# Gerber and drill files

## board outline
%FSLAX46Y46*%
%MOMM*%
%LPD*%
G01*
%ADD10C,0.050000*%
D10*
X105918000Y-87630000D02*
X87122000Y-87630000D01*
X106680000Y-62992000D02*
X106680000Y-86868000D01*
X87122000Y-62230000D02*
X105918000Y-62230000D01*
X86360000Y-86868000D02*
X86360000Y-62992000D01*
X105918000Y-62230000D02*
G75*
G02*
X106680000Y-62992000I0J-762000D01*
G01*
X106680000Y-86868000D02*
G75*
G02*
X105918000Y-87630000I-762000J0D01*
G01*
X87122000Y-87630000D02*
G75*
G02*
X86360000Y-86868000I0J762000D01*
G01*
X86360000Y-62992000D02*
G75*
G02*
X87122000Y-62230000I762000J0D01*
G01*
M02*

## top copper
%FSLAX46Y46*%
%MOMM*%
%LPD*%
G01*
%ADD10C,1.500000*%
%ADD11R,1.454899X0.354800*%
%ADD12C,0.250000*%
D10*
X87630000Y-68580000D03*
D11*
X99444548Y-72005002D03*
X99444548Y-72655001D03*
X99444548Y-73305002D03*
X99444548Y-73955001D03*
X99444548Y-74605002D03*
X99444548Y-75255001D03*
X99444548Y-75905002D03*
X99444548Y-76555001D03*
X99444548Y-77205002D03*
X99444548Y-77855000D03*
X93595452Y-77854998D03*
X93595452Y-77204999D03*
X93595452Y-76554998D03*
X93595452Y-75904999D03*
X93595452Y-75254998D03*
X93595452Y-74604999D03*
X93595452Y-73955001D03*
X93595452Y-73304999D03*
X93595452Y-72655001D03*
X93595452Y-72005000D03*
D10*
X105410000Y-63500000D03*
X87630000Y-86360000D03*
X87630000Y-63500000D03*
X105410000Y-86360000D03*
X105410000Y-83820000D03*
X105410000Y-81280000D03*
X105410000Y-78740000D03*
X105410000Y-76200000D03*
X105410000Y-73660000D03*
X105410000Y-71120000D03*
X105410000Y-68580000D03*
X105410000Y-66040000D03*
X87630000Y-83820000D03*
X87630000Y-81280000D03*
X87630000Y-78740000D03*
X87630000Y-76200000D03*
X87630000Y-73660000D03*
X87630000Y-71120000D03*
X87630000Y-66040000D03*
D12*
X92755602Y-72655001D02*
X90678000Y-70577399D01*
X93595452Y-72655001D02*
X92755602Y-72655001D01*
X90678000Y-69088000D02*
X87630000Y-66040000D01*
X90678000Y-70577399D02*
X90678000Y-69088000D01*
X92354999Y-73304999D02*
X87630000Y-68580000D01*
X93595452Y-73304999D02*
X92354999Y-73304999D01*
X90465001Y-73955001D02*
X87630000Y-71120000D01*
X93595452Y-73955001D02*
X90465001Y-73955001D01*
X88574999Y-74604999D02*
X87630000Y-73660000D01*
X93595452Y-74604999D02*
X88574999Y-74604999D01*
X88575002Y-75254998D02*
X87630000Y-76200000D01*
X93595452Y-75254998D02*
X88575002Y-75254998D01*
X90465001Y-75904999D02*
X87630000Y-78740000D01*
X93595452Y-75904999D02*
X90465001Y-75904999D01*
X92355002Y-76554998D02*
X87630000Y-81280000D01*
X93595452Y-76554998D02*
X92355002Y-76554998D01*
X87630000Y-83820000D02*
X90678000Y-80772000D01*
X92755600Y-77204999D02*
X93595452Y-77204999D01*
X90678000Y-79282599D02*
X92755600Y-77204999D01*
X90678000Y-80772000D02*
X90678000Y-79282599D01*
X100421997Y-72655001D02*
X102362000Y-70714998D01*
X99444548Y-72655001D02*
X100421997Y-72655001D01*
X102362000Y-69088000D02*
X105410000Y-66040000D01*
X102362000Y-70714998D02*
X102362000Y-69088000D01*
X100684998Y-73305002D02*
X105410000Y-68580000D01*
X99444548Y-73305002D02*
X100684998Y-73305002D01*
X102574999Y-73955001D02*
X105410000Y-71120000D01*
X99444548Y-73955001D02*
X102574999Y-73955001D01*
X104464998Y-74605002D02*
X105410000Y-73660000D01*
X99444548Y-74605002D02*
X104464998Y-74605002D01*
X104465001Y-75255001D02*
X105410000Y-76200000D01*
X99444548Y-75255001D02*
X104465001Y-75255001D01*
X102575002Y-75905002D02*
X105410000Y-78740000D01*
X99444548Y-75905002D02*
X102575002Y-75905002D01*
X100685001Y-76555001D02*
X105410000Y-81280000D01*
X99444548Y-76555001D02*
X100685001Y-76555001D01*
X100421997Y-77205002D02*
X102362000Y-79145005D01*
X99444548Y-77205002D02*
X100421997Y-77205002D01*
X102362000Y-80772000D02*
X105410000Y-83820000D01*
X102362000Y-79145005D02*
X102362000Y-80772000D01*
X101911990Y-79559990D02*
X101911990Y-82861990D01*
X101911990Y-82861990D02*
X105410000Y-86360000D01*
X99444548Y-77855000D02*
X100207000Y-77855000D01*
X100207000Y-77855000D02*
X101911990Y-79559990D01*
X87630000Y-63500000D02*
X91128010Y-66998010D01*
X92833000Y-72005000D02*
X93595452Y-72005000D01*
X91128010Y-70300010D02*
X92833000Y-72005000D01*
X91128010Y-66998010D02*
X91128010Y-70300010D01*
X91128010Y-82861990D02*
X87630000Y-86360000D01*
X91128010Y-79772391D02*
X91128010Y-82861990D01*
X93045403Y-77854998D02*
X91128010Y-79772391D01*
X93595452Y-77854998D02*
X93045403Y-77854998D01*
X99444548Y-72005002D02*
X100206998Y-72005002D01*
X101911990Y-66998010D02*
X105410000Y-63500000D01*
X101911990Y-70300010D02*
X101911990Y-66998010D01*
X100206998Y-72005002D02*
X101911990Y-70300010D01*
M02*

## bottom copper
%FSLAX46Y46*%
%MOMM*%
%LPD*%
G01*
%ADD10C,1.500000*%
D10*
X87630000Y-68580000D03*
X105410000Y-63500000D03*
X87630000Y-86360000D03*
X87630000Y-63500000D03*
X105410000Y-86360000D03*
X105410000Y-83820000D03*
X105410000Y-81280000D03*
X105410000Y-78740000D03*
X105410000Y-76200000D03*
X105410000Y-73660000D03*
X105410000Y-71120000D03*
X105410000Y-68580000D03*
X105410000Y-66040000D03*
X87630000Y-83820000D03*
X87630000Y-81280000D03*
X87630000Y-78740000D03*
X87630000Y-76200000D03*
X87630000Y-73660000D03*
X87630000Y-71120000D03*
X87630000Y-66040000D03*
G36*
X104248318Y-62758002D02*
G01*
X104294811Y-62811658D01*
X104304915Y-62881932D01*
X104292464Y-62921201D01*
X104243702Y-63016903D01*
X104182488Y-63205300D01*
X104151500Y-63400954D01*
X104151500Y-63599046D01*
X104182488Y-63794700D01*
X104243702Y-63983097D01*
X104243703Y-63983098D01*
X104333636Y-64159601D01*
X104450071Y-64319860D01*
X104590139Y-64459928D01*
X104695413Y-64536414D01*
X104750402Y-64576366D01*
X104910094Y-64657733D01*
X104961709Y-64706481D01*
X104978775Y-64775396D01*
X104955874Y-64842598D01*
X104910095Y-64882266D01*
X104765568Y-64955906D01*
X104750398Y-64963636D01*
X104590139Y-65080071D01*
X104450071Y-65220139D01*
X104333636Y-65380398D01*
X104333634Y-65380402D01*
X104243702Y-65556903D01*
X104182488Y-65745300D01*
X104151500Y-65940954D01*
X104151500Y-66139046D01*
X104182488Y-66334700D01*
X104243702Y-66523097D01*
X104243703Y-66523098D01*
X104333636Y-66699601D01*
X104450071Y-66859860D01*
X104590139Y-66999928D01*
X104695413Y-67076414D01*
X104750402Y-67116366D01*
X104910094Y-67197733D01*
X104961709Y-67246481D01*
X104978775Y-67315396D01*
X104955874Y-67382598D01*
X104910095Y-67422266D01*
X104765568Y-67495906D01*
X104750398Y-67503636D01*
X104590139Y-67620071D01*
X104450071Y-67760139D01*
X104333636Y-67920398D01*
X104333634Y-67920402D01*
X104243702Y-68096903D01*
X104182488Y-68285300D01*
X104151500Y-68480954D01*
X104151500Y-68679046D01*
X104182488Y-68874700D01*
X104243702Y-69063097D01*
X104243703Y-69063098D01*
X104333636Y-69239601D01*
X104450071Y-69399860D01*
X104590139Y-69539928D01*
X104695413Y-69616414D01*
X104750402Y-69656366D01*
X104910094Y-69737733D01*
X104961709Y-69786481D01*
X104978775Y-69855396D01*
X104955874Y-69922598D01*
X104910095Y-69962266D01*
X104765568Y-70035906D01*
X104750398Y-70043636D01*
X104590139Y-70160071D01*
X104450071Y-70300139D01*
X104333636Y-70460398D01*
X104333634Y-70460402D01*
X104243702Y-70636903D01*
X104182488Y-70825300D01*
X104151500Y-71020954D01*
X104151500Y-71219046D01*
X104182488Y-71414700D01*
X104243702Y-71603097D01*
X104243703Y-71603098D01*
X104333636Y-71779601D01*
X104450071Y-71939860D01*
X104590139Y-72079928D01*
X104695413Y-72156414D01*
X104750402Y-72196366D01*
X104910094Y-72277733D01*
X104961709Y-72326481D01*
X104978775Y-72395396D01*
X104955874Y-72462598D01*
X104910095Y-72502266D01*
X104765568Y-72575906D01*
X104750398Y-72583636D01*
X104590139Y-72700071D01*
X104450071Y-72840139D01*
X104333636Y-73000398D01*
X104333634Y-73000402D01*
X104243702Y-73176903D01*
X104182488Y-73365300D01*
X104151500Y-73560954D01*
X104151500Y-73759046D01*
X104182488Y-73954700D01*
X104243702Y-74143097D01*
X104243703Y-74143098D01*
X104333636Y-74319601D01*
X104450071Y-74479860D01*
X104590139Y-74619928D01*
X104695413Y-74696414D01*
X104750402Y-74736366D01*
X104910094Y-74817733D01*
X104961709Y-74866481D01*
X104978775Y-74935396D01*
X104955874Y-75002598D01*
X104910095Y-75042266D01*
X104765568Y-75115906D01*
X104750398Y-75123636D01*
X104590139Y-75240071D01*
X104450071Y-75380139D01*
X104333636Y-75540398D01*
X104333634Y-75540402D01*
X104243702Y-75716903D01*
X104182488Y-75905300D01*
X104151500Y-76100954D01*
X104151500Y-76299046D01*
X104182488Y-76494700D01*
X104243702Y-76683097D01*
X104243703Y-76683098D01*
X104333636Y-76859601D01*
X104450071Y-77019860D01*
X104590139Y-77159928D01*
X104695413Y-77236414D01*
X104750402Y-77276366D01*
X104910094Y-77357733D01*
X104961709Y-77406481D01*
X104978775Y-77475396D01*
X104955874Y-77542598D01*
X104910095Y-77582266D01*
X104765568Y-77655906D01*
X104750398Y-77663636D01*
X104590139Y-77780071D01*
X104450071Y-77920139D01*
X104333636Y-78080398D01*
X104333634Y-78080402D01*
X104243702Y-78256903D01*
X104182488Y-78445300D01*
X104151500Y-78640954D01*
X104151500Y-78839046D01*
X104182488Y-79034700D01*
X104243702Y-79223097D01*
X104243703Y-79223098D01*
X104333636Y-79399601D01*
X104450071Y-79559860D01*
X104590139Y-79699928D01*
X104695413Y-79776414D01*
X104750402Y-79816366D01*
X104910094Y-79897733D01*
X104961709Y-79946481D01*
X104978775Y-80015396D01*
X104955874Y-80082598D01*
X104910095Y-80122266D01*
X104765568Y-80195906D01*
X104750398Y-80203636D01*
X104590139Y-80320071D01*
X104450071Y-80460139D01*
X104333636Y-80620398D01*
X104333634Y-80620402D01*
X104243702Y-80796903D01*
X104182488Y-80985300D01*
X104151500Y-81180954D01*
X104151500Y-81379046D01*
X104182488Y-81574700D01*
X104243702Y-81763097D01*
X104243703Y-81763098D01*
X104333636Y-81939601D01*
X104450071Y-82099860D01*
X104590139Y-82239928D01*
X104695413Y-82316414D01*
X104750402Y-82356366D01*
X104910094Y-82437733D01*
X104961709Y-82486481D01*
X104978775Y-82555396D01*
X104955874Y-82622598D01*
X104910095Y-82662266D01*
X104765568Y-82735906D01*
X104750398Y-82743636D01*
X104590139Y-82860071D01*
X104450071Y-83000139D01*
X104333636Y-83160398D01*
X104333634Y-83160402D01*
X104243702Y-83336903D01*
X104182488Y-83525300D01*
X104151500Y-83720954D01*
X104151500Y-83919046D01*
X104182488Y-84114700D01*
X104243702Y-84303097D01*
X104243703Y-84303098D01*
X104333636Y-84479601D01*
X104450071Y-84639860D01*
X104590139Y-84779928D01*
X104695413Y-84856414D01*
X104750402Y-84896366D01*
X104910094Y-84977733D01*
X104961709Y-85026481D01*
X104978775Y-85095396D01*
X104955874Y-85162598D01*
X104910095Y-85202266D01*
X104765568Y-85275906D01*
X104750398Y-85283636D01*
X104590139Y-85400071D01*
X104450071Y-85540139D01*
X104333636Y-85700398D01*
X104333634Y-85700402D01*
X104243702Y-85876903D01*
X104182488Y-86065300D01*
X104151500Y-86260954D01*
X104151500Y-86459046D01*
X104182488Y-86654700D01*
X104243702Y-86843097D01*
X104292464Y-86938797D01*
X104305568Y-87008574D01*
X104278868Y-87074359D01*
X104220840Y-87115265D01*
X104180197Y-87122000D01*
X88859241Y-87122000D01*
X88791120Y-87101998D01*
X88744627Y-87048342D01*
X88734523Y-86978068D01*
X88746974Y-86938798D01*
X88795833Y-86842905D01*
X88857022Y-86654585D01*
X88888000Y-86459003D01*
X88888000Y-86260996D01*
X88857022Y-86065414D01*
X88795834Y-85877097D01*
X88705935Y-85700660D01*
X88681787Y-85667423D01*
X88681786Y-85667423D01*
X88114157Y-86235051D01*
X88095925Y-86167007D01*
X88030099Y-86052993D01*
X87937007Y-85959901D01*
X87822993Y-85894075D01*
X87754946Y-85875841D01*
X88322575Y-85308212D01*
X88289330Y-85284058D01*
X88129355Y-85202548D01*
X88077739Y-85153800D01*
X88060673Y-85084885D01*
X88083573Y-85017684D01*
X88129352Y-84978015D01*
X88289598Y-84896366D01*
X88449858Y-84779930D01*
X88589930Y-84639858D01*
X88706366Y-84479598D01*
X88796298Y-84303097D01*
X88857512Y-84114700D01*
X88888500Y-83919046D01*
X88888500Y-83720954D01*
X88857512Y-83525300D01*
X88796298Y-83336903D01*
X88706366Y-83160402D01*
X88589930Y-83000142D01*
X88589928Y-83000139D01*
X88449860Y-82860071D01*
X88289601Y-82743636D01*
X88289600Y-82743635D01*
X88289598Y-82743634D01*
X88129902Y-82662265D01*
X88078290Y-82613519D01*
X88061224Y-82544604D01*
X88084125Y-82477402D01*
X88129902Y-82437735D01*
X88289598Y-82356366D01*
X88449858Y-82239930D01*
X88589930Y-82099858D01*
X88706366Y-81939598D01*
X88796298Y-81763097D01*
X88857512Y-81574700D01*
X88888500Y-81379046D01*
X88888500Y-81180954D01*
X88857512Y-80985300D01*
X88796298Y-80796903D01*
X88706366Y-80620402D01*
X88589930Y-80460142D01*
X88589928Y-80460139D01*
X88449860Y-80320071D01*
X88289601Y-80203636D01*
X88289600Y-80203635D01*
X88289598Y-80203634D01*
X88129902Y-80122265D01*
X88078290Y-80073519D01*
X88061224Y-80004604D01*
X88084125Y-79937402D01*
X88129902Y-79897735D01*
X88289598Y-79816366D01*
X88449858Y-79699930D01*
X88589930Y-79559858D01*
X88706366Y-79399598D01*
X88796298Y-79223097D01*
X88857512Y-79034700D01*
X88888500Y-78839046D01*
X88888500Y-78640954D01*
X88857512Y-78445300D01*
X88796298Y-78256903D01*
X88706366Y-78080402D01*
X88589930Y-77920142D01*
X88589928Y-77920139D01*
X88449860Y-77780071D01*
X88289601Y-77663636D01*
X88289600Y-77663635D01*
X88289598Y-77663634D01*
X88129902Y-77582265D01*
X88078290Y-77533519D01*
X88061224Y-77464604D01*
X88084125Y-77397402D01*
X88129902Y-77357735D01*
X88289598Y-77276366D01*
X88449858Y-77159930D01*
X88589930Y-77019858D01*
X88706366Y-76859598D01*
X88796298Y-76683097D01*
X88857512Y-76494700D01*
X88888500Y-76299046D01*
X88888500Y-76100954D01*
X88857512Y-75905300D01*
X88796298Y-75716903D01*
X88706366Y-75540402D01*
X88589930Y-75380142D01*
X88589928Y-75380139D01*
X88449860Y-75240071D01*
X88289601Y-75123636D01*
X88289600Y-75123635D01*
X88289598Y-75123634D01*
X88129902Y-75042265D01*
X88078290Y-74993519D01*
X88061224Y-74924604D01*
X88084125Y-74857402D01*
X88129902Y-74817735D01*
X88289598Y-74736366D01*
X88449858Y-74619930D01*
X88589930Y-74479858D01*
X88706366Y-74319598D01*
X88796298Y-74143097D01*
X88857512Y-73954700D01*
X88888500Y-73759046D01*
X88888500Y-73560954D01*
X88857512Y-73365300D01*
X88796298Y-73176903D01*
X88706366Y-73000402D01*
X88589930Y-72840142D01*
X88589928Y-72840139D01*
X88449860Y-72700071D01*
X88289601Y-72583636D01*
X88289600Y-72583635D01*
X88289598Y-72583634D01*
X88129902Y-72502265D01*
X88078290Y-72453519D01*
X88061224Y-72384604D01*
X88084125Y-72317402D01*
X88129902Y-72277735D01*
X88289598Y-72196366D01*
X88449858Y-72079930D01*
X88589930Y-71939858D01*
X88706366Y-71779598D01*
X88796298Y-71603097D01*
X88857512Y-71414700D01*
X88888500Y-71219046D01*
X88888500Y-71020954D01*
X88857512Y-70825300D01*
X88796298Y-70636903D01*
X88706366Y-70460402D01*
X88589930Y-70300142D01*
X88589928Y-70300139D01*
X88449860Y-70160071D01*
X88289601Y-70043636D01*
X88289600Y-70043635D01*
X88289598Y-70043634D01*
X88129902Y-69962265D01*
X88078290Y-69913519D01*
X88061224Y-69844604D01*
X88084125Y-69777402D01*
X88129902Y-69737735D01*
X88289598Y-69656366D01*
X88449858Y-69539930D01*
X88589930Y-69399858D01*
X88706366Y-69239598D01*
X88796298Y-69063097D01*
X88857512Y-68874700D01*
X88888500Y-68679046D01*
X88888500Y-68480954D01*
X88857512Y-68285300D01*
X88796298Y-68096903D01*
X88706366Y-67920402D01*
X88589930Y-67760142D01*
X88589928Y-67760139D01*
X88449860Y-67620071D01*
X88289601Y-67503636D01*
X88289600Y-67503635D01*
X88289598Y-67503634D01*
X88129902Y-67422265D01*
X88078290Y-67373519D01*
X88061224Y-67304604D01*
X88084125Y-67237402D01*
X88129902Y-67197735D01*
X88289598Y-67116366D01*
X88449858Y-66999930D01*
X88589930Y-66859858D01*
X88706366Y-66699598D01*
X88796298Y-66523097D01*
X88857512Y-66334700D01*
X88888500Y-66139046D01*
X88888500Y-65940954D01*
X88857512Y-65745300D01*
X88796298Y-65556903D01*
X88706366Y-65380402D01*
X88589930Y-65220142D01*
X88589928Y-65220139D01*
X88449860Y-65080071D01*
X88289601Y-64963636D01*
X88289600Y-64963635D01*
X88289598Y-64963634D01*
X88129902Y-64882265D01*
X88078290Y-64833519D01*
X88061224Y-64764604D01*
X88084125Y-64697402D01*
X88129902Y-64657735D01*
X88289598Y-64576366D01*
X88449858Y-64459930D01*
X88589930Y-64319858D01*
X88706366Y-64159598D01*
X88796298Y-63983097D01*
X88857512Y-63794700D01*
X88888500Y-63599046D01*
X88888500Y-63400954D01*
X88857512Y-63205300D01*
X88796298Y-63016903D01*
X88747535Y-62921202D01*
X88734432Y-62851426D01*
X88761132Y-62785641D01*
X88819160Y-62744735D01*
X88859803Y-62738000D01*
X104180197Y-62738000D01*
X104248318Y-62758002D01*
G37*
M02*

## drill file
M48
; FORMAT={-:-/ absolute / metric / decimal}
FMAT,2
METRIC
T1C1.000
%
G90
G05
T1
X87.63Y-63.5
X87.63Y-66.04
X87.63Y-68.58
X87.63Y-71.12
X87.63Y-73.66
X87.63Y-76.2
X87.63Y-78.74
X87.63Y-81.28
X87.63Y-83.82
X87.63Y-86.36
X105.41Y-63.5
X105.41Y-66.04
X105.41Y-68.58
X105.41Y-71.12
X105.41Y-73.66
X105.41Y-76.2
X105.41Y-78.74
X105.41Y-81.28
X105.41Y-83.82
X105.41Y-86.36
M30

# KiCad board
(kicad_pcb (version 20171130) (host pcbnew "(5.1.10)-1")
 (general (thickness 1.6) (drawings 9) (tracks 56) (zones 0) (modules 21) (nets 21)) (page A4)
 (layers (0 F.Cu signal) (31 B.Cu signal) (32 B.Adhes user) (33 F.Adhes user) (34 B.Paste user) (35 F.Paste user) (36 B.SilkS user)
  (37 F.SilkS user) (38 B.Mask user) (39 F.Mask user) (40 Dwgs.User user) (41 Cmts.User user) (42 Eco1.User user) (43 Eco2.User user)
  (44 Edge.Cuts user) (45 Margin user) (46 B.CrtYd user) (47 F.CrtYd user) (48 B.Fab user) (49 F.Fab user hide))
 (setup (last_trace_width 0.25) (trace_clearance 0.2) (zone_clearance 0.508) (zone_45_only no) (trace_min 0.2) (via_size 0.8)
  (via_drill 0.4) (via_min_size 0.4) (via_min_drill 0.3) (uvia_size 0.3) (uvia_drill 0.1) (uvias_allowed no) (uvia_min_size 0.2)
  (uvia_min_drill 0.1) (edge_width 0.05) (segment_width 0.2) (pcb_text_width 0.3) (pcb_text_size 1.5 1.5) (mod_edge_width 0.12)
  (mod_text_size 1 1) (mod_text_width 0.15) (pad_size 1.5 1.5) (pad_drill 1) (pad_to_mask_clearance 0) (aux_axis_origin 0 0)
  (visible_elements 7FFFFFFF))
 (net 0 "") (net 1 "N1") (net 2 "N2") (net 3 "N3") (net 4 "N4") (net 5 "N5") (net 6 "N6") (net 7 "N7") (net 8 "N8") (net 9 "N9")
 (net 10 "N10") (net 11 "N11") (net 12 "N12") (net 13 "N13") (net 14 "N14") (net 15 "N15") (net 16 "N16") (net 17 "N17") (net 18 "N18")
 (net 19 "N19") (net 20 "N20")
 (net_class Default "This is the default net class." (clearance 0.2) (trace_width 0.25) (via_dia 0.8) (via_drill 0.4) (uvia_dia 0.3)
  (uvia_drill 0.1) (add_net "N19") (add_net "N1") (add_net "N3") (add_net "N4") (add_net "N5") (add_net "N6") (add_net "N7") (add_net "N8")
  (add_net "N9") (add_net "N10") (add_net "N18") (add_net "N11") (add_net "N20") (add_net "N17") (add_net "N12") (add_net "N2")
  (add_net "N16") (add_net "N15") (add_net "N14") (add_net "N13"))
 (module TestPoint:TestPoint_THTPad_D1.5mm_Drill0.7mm (layer F.Cu) (at 87.63 68.58)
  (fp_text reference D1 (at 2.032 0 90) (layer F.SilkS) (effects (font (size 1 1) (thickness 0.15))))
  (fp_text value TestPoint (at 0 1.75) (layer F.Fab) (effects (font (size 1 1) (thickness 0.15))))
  (pad 1 thru_hole circle (at 0 0) (size 1.5 1.5) (drill 1) (layers *.Cu *.Mask) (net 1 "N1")))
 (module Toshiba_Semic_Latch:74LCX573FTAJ (layer F.Cu) (at 96.52 74.93)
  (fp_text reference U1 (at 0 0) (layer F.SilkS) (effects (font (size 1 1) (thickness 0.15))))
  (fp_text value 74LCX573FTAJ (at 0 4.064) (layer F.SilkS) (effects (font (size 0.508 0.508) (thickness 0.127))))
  (pad 20 smd rect (at 2.924548 -2.924998) (size 1.454899 0.3548) (layers F.Cu F.Paste F.Mask) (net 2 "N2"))
  (pad 19 smd rect (at 2.924548 -2.274999) (size 1.454899 0.3548) (layers F.Cu F.Paste F.Mask) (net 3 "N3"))
  (pad 18 smd rect (at 2.924548 -1.624998) (size 1.454899 0.3548) (layers F.Cu F.Paste F.Mask) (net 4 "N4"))
  (pad 17 smd rect (at 2.924548 -0.974999) (size 1.454899 0.3548) (layers F.Cu F.Paste F.Mask) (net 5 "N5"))
  (pad 16 smd rect (at 2.924548 -0.324998) (size 1.454899 0.3548) (layers F.Cu F.Paste F.Mask) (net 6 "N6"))
  (pad 15 smd rect (at 2.924548 0.325001) (size 1.454899 0.3548) (layers F.Cu F.Paste F.Mask) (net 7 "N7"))
  (pad 14 smd rect (at 2.924548 0.975002) (size 1.454899 0.3548) (layers F.Cu F.Paste F.Mask) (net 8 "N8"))
  (pad 13 smd rect (at 2.924548 1.625001) (size 1.454899 0.3548) (layers F.Cu F.Paste F.Mask) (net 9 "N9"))
  (pad 12 smd rect (at 2.924548 2.275002) (size 1.454899 0.3548) (layers F.Cu F.Paste F.Mask) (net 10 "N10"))
  (pad 11 smd rect (at 2.924548 2.925) (size 1.454899 0.3548) (layers F.Cu F.Paste F.Mask) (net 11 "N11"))
  (pad 10 smd rect (at -2.924548 2.924998) (size 1.454899 0.3548) (layers F.Cu F.Paste F.Mask) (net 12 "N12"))
  (pad 9 smd rect (at -2.924548 2.274999) (size 1.454899 0.3548) (layers F.Cu F.Paste F.Mask) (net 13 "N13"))
  (pad 8 smd rect (at -2.924548 1.624998) (size 1.454899 0.3548) (layers F.Cu F.Paste F.Mask) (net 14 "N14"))
  (pad 7 smd rect (at -2.924548 0.974999) (size 1.454899 0.3548) (layers F.Cu F.Paste F.Mask) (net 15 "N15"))
  (pad 6 smd rect (at -2.924548 0.324998) (size 1.454899 0.3548) (layers F.Cu F.Paste F.Mask) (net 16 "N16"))
  (pad 5 smd rect (at -2.924548 -0.325001) (size 1.454899 0.3548) (layers F.Cu F.Paste F.Mask) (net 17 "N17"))
  (pad 4 smd rect (at -2.924548 -0.974999) (size 1.454899 0.3548) (layers F.Cu F.Paste F.Mask) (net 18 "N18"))
  (pad 3 smd rect (at -2.924548 -1.625001) (size 1.454899 0.3548) (layers F.Cu F.Paste F.Mask) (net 1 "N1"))
  (pad 2 smd rect (at -2.924548 -2.274999) (size 1.454899 0.3548) (layers F.Cu F.Paste F.Mask) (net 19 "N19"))
  (pad 1 smd rect (at -2.924548 -2.925) (size 1.454899 0.3548) (layers F.Cu F.Paste F.Mask) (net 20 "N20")))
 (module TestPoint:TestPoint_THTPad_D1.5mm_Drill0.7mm (layer F.Cu) (at 105.41 63.5)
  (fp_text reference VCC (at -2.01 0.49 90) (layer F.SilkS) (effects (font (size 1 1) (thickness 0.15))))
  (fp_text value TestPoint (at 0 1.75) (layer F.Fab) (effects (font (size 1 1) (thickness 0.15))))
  (pad 1 thru_hole circle (at 0 0) (size 1.5 1.5) (drill 1) (layers *.Cu *.Mask) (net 2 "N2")))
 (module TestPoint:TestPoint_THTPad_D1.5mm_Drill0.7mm (layer F.Cu) (at 87.63 86.36)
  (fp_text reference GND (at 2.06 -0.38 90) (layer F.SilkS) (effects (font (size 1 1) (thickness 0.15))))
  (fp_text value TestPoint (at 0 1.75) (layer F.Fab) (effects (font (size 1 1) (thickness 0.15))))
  (pad 1 thru_hole circle (at 0 0) (size 1.5 1.5) (drill 1) (layers *.Cu *.Mask) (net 12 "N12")))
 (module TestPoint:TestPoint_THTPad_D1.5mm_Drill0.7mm (layer F.Cu) (at 87.63 63.5)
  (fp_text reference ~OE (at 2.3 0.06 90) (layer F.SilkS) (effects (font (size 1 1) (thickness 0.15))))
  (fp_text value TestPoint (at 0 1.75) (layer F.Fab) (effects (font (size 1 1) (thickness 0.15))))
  (pad 1 thru_hole circle (at 0 0) (size 1.5 1.5) (drill 1) (layers *.Cu *.Mask) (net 20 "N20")))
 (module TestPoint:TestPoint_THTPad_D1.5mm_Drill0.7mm (layer F.Cu) (at 105.41 86.36)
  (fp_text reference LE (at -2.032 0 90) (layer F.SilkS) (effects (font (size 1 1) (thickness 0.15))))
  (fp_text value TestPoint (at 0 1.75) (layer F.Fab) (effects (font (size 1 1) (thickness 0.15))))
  (pad 1 thru_hole circle (at 0 0) (size 1.5 1.5) (drill 1) (layers *.Cu *.Mask) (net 11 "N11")))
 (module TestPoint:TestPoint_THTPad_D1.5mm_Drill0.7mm (layer F.Cu) (at 105.41 83.82)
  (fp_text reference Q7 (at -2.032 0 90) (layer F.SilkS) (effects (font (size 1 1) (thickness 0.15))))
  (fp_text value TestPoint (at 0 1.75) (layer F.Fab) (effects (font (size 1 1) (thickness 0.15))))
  (pad 1 thru_hole circle (at 0 0) (size 1.5 1.5) (drill 1) (layers *.Cu *.Mask) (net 10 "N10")))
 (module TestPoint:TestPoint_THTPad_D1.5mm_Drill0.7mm (layer F.Cu) (at 105.41 81.28)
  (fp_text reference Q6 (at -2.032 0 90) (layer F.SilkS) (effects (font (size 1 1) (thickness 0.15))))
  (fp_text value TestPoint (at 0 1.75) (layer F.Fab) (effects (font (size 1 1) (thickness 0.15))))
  (pad 1 thru_hole circle (at 0 0) (size 1.5 1.5) (drill 1) (layers *.Cu *.Mask) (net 9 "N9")))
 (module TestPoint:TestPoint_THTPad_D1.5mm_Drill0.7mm (layer F.Cu) (at 105.41 78.74)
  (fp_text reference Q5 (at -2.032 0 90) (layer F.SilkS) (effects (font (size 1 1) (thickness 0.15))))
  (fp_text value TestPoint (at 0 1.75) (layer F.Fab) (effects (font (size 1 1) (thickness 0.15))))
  (pad 1 thru_hole circle (at 0 0) (size 1.5 1.5) (drill 1) (layers *.Cu *.Mask) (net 8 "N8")))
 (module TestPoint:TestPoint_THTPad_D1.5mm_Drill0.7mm (layer F.Cu) (at 105.41 76.2)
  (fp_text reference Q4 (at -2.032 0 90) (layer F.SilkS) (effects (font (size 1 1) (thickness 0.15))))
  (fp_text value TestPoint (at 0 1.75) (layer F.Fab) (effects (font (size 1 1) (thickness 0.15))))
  (pad 1 thru_hole circle (at 0 0) (size 1.5 1.5) (drill 1) (layers *.Cu *.Mask) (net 7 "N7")))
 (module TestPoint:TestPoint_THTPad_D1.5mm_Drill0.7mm (layer F.Cu) (at 105.41 73.66)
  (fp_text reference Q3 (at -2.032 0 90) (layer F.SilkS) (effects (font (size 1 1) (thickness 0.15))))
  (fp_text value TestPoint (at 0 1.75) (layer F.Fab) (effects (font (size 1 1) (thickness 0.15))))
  (pad 1 thru_hole circle (at 0 0) (size 1.5 1.5) (drill 1) (layers *.Cu *.Mask) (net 6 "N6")))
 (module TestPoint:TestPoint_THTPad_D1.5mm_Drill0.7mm (layer F.Cu) (at 105.41 71.12)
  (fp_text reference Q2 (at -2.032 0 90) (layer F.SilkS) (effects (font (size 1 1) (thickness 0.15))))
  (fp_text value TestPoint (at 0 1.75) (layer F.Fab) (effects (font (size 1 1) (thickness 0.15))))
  (pad 1 thru_hole circle (at 0 0) (size 1.5 1.5) (drill 1) (layers *.Cu *.Mask) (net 5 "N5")))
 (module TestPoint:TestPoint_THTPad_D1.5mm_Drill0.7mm (layer F.Cu) (at 105.41 68.58)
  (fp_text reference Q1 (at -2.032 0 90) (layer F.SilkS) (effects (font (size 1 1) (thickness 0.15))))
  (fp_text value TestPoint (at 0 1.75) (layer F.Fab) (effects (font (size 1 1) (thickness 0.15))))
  (pad 1 thru_hole circle (at 0 0) (size 1.5 1.5) (drill 1) (layers *.Cu *.Mask) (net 4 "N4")))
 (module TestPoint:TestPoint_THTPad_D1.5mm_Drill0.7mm (layer F.Cu) (at 105.41 66.04)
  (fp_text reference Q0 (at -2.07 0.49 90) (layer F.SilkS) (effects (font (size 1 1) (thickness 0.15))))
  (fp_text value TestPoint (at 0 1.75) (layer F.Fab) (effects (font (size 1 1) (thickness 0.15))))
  (pad 1 thru_hole circle (at 0 0) (size 1.5 1.5) (drill 1) (layers *.Cu *.Mask) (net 3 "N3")))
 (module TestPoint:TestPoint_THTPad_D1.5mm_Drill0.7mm (layer F.Cu) (at 87.63 83.82)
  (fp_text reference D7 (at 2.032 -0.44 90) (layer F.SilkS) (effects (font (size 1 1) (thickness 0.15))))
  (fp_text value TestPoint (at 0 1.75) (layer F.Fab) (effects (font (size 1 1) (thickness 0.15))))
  (pad 1 thru_hole circle (at 0 0) (size 1.5 1.5) (drill 1) (layers *.Cu *.Mask) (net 13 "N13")))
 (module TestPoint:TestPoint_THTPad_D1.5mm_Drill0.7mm (layer F.Cu) (at 87.63 81.28)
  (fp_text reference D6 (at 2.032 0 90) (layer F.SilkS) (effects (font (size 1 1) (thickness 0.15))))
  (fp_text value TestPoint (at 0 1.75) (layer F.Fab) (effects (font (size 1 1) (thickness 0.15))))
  (pad 1 thru_hole circle (at 0 0) (size 1.5 1.5) (drill 1) (layers *.Cu *.Mask) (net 14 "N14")))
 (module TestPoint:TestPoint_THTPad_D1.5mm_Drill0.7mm (layer F.Cu) (at 87.63 78.74)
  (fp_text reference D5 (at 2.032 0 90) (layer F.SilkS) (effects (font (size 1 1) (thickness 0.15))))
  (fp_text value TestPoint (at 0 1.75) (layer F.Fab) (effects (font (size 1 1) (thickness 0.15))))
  (pad 1 thru_hole circle (at 0 0) (size 1.5 1.5) (drill 1) (layers *.Cu *.Mask) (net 15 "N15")))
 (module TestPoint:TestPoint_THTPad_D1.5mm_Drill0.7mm (layer F.Cu) (at 87.63 76.2)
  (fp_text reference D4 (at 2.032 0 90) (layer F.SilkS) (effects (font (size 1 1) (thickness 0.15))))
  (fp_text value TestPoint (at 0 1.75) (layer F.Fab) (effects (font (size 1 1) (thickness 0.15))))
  (pad 1 thru_hole circle (at 0 0) (size 1.5 1.5) (drill 1) (layers *.Cu *.Mask) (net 16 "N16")))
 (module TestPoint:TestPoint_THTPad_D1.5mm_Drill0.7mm (layer F.Cu) (at 87.63 73.66)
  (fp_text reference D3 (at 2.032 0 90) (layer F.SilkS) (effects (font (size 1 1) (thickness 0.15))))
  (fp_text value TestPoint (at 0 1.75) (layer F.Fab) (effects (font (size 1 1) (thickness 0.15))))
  (pad 1 thru_hole circle (at 0 0) (size 1.5 1.5) (drill 1) (layers *.Cu *.Mask) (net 17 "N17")))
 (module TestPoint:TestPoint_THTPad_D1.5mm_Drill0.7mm (layer F.Cu) (at 87.63 71.12)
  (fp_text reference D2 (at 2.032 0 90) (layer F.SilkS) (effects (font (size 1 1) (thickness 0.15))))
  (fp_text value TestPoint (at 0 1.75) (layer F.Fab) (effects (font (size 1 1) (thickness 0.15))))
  (pad 1 thru_hole circle (at 0 0) (size 1.5 1.5) (drill 1) (layers *.Cu *.Mask) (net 18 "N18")))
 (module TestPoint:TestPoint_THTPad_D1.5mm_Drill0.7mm (layer F.Cu) (at 87.63 66.04)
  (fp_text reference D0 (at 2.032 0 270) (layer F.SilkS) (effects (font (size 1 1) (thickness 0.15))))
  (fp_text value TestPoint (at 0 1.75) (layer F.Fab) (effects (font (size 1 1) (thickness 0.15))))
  (pad 1 thru_hole circle (at 0 0) (size 1.5 1.5) (drill 1) (layers *.Cu *.Mask) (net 19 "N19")))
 (gr_line (start 105.918 87.63) (end 87.122 87.63) (layer Edge.Cuts) (width 0.05))
 (gr_line (start 106.68 62.992) (end 106.68 86.868) (layer Edge.Cuts) (width 0.05))
 (gr_line (start 87.122 62.23) (end 105.918 62.23) (layer Edge.Cuts) (width 0.05))
 (gr_line (start 86.36 86.868) (end 86.36 62.992) (layer Edge.Cuts) (width 0.05))
 (gr_arc (start 105.918 62.992) (end 106.68 62.992) (angle -90) (layer Edge.Cuts) (width 0.05))
 (gr_arc (start 105.918 86.868) (end 105.918 87.63) (angle -90) (layer Edge.Cuts) (width 0.05))
 (gr_arc (start 87.122 86.868) (end 86.36 86.868) (angle -90) (layer Edge.Cuts) (width 0.05))
 (gr_arc (start 87.122 62.992) (end 87.122 62.23) (angle -90) (layer Edge.Cuts) (width 0.05))
 (segment (start 92.755602 72.655001) (end 90.678 70.577399) (width 0.25) (layer F.Cu) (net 19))
 (segment (start 93.595452 72.655001) (end 92.755602 72.655001) (width 0.25) (layer F.Cu) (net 19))
 (segment (start 90.678 69.088) (end 87.63 66.04) (width 0.25) (layer F.Cu) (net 19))
 (segment (start 90.678 70.577399) (end 90.678 69.088) (width 0.25) (layer F.Cu) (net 19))
 (segment (start 92.354999 73.304999) (end 87.63 68.58) (width 0.25) (layer F.Cu) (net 1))
 (segment (start 93.595452 73.304999) (end 92.354999 73.304999) (width 0.25) (layer F.Cu) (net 1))
 (segment (start 90.465001 73.955001) (end 87.63 71.12) (width 0.25) (layer F.Cu) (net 18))
 (segment (start 93.595452 73.955001) (end 90.465001 73.955001) (width 0.25) (layer F.Cu) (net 18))
 (segment (start 88.574999 74.604999) (end 87.63 73.66) (width 0.25) (layer F.Cu) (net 17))
 (segment (start 93.595452 74.604999) (end 88.574999 74.604999) (width 0.25) (layer F.Cu) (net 17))
 (segment (start 88.575002 75.254998) (end 87.63 76.2) (width 0.25) (layer F.Cu) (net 16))
 (segment (start 93.595452 75.254998) (end 88.575002 75.254998) (width 0.25) (layer F.Cu) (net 16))
 (segment (start 90.465001 75.904999) (end 87.63 78.74) (width 0.25) (layer F.Cu) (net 15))
 (segment (start 93.595452 75.904999) (end 90.465001 75.904999) (width 0.25) (layer F.Cu) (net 15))
 (segment (start 92.355002 76.554998) (end 87.63 81.28) (width 0.25) (layer F.Cu) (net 14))
 (segment (start 93.595452 76.554998) (end 92.355002 76.554998) (width 0.25) (layer F.Cu) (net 14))
 (segment (start 87.63 83.82) (end 90.678 80.772) (width 0.25) (layer F.Cu) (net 13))
 (segment (start 92.7556 77.204999) (end 93.595452 77.204999) (width 0.25) (layer F.Cu) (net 13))
 (segment (start 90.678 79.282599) (end 92.7556 77.204999) (width 0.25) (layer F.Cu) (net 13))
 (segment (start 90.678 80.772) (end 90.678 79.282599) (width 0.25) (layer F.Cu) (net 13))
 (segment (start 100.421997 72.655001) (end 102.362 70.714998) (width 0.25) (layer F.Cu) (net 3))
 (segment (start 99.444548 72.655001) (end 100.421997 72.655001) (width 0.25) (layer F.Cu) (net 3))
 (segment (start 102.362 69.088) (end 105.41 66.04) (width 0.25) (layer F.Cu) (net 3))
 (segment (start 102.362 70.714998) (end 102.362 69.088) (width 0.25) (layer F.Cu) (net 3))
 (segment (start 100.684998 73.305002) (end 105.41 68.58) (width 0.25) (layer F.Cu) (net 4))
 (segment (start 99.444548 73.305002) (end 100.684998 73.305002) (width 0.25) (layer F.Cu) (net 4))
 (segment (start 102.574999 73.955001) (end 105.41 71.12) (width 0.25) (layer F.Cu) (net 5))
 (segment (start 99.444548 73.955001) (end 102.574999 73.955001) (width 0.25) (layer F.Cu) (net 5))
 (segment (start 104.464998 74.605002) (end 105.41 73.66) (width 0.25) (layer F.Cu) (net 6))
 (segment (start 99.444548 74.605002) (end 104.464998 74.605002) (width 0.25) (layer F.Cu) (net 6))
 (segment (start 104.465001 75.255001) (end 105.41 76.2) (width 0.25) (layer F.Cu) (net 7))
 (segment (start 99.444548 75.255001) (end 104.465001 75.255001) (width 0.25) (layer F.Cu) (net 7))
 (segment (start 102.575002 75.905002) (end 105.41 78.74) (width 0.25) (layer F.Cu) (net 8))
 (segment (start 99.444548 75.905002) (end 102.575002 75.905002) (width 0.25) (layer F.Cu) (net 8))
 (segment (start 100.685001 76.555001) (end 105.41 81.28) (width 0.25) (layer F.Cu) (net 9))
 (segment (start 99.444548 76.555001) (end 100.685001 76.555001) (width 0.25) (layer F.Cu) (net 9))
 (segment (start 100.421997 77.205002) (end 102.362 79.145005) (width 0.25) (layer F.Cu) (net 10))
 (segment (start 99.444548 77.205002) (end 100.421997 77.205002) (width 0.25) (layer F.Cu) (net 10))
 (segment (start 102.362 80.772) (end 105.41 83.82) (width 0.25) (layer F.Cu) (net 10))
 (segment (start 102.362 79.145005) (end 102.362 80.772) (width 0.25) (layer F.Cu) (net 10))
 (segment (start 101.91199 79.55999) (end 101.91199 82.86199) (width 0.25) (layer F.Cu) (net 11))
 (segment (start 101.91199 82.86199) (end 105.41 86.36) (width 0.25) (layer F.Cu) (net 11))
 (segment (start 99.444548 77.855) (end 100.207 77.855) (width 0.25) (layer F.Cu) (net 11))
 (segment (start 100.207 77.855) (end 101.91199 79.55999) (width 0.25) (layer F.Cu) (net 11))
 (segment (start 87.63 63.5) (end 91.12801 66.99801) (width 0.25) (layer F.Cu) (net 20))
 (segment (start 92.833 72.005) (end 93.595452 72.005) (width 0.25) (layer F.Cu) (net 20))
 (segment (start 91.12801 70.30001) (end 92.833 72.005) (width 0.25) (layer F.Cu) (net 20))
 (segment (start 91.12801 66.99801) (end 91.12801 70.30001) (width 0.25) (layer F.Cu) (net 20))
 (segment (start 91.12801 82.86199) (end 87.63 86.36) (width 0.25) (layer F.Cu) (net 12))
 (segment (start 91.12801 79.772391) (end 91.12801 82.86199) (width 0.25) (layer F.Cu) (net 12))
 (segment (start 93.045403 77.854998) (end 91.12801 79.772391) (width 0.25) (layer F.Cu) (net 12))
 (segment (start 93.595452 77.854998) (end 93.045403 77.854998) (width 0.25) (layer F.Cu) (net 12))
 (segment (start 99.444548 72.005002) (end 100.206998 72.005002) (width 0.25) (layer F.Cu) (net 2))
 (segment (start 101.91199 66.99801) (end 105.41 63.5) (width 0.25) (layer F.Cu) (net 2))
 (segment (start 101.91199 70.30001) (end 101.91199 66.99801) (width 0.25) (layer F.Cu) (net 2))
 (segment (start 100.206998 72.005002) (end 101.91199 70.30001) (width 0.25) (layer F.Cu) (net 2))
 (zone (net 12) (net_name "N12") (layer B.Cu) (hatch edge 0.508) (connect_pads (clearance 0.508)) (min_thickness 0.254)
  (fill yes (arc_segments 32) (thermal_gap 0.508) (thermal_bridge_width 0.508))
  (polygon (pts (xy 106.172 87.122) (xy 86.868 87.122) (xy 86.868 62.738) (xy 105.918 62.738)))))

